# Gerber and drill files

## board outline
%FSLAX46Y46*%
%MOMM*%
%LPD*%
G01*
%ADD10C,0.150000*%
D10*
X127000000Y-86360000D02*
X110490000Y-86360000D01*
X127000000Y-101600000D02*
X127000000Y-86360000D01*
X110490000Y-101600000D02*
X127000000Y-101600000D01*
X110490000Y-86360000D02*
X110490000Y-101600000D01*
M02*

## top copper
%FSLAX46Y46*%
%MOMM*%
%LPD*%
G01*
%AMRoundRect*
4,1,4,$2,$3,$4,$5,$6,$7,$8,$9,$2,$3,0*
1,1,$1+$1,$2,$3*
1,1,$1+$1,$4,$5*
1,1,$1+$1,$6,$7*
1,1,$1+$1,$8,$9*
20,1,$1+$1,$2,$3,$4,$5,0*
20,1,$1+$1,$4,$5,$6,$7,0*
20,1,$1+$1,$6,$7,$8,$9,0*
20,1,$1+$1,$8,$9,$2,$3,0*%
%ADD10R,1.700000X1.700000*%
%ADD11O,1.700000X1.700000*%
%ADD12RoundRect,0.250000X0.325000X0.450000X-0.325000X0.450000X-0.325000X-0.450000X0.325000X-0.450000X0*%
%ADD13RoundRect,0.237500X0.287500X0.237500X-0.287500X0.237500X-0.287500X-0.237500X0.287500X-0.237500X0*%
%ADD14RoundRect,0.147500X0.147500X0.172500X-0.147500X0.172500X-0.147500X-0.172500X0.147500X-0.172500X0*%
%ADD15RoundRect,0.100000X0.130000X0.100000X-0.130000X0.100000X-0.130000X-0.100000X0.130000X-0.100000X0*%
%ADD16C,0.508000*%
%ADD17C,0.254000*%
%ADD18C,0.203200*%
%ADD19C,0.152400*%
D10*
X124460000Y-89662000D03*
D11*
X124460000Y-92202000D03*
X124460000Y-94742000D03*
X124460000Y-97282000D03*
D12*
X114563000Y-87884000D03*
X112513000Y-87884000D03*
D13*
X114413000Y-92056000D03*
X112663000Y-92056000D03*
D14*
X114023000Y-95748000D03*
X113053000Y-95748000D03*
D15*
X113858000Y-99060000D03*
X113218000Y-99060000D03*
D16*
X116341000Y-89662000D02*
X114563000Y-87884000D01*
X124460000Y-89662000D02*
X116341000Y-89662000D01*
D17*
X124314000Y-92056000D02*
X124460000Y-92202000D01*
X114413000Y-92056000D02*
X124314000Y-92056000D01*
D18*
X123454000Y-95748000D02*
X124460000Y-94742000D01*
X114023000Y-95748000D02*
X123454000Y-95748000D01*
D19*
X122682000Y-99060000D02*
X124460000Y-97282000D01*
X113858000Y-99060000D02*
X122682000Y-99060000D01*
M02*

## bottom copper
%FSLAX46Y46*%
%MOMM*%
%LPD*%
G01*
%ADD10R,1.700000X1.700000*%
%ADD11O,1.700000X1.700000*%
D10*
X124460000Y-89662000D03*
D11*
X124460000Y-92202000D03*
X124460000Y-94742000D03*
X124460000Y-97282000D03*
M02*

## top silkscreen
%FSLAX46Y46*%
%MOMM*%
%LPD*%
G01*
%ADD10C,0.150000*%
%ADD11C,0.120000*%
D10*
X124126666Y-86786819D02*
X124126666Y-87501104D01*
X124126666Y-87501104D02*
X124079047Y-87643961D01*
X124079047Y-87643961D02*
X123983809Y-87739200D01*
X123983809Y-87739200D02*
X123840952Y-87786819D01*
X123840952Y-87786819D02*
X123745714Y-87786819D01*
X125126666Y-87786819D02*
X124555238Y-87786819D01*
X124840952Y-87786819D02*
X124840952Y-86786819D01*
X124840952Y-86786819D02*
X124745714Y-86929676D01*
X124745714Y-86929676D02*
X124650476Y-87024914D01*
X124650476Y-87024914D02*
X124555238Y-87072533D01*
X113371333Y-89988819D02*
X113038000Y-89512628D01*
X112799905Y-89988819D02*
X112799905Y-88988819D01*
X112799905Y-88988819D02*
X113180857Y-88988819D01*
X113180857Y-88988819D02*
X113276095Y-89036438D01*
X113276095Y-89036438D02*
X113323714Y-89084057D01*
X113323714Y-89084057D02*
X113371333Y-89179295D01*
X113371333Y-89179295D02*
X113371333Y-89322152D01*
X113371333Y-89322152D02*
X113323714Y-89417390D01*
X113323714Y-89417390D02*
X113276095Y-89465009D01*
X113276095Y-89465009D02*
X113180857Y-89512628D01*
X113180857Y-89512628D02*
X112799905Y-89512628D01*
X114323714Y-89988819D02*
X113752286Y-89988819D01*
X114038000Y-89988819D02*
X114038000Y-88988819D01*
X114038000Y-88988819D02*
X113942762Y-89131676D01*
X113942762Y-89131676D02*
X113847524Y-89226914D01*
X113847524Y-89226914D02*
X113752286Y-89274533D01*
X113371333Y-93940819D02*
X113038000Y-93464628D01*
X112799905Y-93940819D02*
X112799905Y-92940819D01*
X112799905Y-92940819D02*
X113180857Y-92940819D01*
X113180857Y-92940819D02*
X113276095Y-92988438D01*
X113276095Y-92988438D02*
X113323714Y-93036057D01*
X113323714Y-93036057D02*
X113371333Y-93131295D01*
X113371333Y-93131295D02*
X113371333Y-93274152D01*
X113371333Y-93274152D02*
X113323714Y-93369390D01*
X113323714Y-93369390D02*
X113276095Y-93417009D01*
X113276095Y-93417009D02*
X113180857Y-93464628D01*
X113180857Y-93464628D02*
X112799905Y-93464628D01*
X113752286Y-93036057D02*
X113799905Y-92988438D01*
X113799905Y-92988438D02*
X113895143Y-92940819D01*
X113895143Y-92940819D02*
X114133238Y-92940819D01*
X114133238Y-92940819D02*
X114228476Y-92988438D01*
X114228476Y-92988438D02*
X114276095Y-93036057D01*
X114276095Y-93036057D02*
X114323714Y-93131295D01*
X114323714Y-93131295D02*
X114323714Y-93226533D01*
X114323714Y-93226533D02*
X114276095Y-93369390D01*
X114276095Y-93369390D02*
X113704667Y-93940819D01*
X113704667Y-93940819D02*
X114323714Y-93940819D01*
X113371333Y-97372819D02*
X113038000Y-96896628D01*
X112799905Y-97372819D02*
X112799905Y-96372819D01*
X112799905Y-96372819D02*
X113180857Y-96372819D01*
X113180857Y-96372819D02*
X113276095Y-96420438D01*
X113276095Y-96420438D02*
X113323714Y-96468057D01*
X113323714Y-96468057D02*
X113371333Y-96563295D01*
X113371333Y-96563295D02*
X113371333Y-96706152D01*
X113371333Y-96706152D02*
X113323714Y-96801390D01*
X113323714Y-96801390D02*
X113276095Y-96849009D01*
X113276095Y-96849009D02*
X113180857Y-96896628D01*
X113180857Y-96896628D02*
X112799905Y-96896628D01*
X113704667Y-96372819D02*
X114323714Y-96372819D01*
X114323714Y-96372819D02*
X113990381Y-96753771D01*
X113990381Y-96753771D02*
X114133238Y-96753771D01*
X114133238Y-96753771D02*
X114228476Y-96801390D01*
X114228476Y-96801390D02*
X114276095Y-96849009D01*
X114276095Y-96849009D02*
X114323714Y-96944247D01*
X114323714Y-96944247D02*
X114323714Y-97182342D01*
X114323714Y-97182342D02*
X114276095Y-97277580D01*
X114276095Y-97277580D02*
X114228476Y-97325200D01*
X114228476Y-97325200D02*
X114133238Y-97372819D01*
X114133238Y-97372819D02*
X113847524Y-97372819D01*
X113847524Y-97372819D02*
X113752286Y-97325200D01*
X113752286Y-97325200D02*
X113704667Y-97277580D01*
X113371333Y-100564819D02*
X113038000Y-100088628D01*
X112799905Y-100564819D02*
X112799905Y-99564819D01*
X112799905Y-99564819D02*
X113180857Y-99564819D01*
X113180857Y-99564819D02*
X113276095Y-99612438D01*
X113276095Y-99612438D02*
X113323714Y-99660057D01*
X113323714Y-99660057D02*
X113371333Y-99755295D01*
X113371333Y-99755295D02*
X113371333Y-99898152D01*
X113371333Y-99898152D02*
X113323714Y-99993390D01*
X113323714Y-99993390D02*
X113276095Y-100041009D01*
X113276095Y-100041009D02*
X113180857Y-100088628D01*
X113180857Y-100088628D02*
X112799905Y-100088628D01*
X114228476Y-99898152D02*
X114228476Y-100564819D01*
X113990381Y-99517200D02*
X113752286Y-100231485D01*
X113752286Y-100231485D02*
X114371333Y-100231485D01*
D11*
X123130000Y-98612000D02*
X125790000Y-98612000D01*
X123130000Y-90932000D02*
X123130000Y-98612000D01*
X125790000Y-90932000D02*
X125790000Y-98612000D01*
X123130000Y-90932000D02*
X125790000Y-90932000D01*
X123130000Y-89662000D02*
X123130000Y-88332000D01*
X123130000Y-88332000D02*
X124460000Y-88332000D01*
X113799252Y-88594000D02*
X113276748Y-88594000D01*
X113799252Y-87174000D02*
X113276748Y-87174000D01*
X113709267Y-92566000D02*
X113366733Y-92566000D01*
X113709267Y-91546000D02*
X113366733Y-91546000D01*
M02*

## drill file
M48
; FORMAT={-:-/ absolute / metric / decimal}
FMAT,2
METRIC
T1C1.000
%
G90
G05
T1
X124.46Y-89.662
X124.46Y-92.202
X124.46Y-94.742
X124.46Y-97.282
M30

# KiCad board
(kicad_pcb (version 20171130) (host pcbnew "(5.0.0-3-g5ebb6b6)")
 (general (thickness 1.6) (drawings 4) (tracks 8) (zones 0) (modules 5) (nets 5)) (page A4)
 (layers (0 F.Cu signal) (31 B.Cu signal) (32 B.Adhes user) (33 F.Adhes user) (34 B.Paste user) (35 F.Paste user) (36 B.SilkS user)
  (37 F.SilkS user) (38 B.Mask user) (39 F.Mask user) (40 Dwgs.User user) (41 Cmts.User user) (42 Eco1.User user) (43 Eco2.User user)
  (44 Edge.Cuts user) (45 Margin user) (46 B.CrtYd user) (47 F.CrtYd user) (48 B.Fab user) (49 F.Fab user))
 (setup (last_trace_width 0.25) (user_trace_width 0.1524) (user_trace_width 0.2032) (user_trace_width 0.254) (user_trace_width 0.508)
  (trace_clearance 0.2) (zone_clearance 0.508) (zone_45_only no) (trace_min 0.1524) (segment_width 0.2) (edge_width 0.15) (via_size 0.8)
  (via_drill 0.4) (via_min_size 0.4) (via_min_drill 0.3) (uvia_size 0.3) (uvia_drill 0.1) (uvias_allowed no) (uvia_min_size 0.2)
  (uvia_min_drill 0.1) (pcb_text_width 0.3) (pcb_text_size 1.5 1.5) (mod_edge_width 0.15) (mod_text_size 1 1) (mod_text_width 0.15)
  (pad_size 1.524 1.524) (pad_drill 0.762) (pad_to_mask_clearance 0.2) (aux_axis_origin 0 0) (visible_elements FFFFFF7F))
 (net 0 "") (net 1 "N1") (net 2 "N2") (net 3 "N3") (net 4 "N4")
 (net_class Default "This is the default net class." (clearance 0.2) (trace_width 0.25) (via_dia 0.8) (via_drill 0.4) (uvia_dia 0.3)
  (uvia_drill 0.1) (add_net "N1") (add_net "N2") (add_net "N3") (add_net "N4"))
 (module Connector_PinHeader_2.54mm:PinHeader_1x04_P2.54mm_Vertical (layer F.Cu) (at 124.46 89.662)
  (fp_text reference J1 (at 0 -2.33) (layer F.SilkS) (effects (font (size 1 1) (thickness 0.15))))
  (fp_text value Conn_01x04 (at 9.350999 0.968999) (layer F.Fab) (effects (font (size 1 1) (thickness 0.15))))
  (fp_line (start -1.33 8.95) (end 1.33 8.95) (layer F.SilkS) (width 0.12))
  (fp_line (start -1.33 1.27) (end -1.33 8.95) (layer F.SilkS) (width 0.12))
  (fp_line (start 1.33 1.27) (end 1.33 8.95) (layer F.SilkS) (width 0.12))
  (fp_line (start -1.33 1.27) (end 1.33 1.27) (layer F.SilkS) (width 0.12))
  (fp_line (start -1.33 0) (end -1.33 -1.33) (layer F.SilkS) (width 0.12))
  (fp_line (start -1.33 -1.33) (end 0 -1.33) (layer F.SilkS) (width 0.12))
  (pad 1 thru_hole rect (at 0 0) (size 1.7 1.7) (drill 1) (layers *.Cu *.Mask) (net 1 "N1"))
  (pad 2 thru_hole oval (at 0 2.54) (size 1.7 1.7) (drill 1) (layers *.Cu *.Mask) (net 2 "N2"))
  (pad 3 thru_hole oval (at 0 5.08) (size 1.7 1.7) (drill 1) (layers *.Cu *.Mask) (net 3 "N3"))
  (pad 4 thru_hole oval (at 0 7.62) (size 1.7 1.7) (drill 1) (layers *.Cu *.Mask) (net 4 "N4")))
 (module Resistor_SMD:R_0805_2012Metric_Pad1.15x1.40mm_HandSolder (layer F.Cu) (at 113.538 87.884 180)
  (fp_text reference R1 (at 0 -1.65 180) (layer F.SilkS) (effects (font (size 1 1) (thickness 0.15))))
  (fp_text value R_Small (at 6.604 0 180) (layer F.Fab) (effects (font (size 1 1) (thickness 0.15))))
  (fp_line (start -0.261252 -0.71) (end 0.261252 -0.71) (layer F.SilkS) (width 0.12))
  (fp_line (start -0.261252 0.71) (end 0.261252 0.71) (layer F.SilkS) (width 0.12))
  (pad 1 smd roundrect (at -1.025 0 180) (size 1.15 1.4) (layers F.Cu F.Paste F.Mask) (roundrect_rratio 0.217391) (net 1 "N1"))
  (pad 2 smd roundrect (at 1.025 0 180) (size 1.15 1.4) (layers F.Cu F.Paste F.Mask) (roundrect_rratio 0.217391)))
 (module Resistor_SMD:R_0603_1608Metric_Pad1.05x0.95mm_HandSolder (layer F.Cu) (at 113.538 92.056 180)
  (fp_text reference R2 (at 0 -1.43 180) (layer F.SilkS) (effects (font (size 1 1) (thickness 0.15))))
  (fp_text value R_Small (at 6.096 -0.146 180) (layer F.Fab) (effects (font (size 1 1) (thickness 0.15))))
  (fp_line (start -0.171267 -0.51) (end 0.171267 -0.51) (layer F.SilkS) (width 0.12))
  (fp_line (start -0.171267 0.51) (end 0.171267 0.51) (layer F.SilkS) (width 0.12))
  (pad 1 smd roundrect (at -0.875 0 180) (size 1.05 0.95) (layers F.Cu F.Paste F.Mask) (roundrect_rratio 0.25) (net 2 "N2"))
  (pad 2 smd roundrect (at 0.875 0 180) (size 1.05 0.95) (layers F.Cu F.Paste F.Mask) (roundrect_rratio 0.25)))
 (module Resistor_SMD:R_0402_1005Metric (layer F.Cu) (at 113.538 95.748 180)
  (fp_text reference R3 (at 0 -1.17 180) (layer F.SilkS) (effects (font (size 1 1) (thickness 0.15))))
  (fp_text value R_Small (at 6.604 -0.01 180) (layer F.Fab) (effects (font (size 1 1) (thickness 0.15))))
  (pad 1 smd roundrect (at -0.485 0 180) (size 0.59 0.64) (layers F.Cu F.Paste F.Mask) (roundrect_rratio 0.25) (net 3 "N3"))
  (pad 2 smd roundrect (at 0.485 0 180) (size 0.59 0.64) (layers F.Cu F.Paste F.Mask) (roundrect_rratio 0.25)))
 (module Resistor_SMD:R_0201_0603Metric (layer F.Cu) (at 113.538 99.06 180)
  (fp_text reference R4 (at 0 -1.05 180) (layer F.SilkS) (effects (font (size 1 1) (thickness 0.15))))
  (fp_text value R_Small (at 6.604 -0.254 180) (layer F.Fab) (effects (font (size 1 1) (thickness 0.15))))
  (pad "" smd roundrect (at -0.345 0 180) (size 0.318 0.36) (layers F.Paste) (roundrect_rratio 0.25))
  (pad "" smd roundrect (at 0.345 0 180) (size 0.318 0.36) (layers F.Paste) (roundrect_rratio 0.25))
  (pad 1 smd roundrect (at -0.32 0 180) (size 0.46 0.4) (layers F.Cu F.Mask) (roundrect_rratio 0.25) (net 4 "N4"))
  (pad 2 smd roundrect (at 0.32 0 180) (size 0.46 0.4) (layers F.Cu F.Mask) (roundrect_rratio 0.25)))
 (gr_line (start 127 86.36) (end 110.49 86.36) (layer Edge.Cuts) (width 0.15))
 (gr_line (start 127 101.6) (end 127 86.36) (layer Edge.Cuts) (width 0.15))
 (gr_line (start 110.49 101.6) (end 127 101.6) (layer Edge.Cuts) (width 0.15))
 (gr_line (start 110.49 86.36) (end 110.49 101.6) (layer Edge.Cuts) (width 0.15))
 (segment (start 116.341 89.662) (end 114.563 87.884) (width 0.508) (layer F.Cu) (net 1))
 (segment (start 124.46 89.662) (end 116.341 89.662) (width 0.508) (layer F.Cu) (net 1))
 (segment (start 124.314 92.056) (end 124.46 92.202) (width 0.254) (layer F.Cu) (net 2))
 (segment (start 114.413 92.056) (end 124.314 92.056) (width 0.254) (layer F.Cu) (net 2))
 (segment (start 123.454 95.748) (end 124.46 94.742) (width 0.2032) (layer F.Cu) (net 3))
 (segment (start 114.023 95.748) (end 123.454 95.748) (width 0.2032) (layer F.Cu) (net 3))
 (segment (start 122.682 99.06) (end 124.46 97.282) (width 0.1524) (layer F.Cu) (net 4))
 (segment (start 113.858 99.06) (end 122.682 99.06) (width 0.1524) (layer F.Cu) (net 4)))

